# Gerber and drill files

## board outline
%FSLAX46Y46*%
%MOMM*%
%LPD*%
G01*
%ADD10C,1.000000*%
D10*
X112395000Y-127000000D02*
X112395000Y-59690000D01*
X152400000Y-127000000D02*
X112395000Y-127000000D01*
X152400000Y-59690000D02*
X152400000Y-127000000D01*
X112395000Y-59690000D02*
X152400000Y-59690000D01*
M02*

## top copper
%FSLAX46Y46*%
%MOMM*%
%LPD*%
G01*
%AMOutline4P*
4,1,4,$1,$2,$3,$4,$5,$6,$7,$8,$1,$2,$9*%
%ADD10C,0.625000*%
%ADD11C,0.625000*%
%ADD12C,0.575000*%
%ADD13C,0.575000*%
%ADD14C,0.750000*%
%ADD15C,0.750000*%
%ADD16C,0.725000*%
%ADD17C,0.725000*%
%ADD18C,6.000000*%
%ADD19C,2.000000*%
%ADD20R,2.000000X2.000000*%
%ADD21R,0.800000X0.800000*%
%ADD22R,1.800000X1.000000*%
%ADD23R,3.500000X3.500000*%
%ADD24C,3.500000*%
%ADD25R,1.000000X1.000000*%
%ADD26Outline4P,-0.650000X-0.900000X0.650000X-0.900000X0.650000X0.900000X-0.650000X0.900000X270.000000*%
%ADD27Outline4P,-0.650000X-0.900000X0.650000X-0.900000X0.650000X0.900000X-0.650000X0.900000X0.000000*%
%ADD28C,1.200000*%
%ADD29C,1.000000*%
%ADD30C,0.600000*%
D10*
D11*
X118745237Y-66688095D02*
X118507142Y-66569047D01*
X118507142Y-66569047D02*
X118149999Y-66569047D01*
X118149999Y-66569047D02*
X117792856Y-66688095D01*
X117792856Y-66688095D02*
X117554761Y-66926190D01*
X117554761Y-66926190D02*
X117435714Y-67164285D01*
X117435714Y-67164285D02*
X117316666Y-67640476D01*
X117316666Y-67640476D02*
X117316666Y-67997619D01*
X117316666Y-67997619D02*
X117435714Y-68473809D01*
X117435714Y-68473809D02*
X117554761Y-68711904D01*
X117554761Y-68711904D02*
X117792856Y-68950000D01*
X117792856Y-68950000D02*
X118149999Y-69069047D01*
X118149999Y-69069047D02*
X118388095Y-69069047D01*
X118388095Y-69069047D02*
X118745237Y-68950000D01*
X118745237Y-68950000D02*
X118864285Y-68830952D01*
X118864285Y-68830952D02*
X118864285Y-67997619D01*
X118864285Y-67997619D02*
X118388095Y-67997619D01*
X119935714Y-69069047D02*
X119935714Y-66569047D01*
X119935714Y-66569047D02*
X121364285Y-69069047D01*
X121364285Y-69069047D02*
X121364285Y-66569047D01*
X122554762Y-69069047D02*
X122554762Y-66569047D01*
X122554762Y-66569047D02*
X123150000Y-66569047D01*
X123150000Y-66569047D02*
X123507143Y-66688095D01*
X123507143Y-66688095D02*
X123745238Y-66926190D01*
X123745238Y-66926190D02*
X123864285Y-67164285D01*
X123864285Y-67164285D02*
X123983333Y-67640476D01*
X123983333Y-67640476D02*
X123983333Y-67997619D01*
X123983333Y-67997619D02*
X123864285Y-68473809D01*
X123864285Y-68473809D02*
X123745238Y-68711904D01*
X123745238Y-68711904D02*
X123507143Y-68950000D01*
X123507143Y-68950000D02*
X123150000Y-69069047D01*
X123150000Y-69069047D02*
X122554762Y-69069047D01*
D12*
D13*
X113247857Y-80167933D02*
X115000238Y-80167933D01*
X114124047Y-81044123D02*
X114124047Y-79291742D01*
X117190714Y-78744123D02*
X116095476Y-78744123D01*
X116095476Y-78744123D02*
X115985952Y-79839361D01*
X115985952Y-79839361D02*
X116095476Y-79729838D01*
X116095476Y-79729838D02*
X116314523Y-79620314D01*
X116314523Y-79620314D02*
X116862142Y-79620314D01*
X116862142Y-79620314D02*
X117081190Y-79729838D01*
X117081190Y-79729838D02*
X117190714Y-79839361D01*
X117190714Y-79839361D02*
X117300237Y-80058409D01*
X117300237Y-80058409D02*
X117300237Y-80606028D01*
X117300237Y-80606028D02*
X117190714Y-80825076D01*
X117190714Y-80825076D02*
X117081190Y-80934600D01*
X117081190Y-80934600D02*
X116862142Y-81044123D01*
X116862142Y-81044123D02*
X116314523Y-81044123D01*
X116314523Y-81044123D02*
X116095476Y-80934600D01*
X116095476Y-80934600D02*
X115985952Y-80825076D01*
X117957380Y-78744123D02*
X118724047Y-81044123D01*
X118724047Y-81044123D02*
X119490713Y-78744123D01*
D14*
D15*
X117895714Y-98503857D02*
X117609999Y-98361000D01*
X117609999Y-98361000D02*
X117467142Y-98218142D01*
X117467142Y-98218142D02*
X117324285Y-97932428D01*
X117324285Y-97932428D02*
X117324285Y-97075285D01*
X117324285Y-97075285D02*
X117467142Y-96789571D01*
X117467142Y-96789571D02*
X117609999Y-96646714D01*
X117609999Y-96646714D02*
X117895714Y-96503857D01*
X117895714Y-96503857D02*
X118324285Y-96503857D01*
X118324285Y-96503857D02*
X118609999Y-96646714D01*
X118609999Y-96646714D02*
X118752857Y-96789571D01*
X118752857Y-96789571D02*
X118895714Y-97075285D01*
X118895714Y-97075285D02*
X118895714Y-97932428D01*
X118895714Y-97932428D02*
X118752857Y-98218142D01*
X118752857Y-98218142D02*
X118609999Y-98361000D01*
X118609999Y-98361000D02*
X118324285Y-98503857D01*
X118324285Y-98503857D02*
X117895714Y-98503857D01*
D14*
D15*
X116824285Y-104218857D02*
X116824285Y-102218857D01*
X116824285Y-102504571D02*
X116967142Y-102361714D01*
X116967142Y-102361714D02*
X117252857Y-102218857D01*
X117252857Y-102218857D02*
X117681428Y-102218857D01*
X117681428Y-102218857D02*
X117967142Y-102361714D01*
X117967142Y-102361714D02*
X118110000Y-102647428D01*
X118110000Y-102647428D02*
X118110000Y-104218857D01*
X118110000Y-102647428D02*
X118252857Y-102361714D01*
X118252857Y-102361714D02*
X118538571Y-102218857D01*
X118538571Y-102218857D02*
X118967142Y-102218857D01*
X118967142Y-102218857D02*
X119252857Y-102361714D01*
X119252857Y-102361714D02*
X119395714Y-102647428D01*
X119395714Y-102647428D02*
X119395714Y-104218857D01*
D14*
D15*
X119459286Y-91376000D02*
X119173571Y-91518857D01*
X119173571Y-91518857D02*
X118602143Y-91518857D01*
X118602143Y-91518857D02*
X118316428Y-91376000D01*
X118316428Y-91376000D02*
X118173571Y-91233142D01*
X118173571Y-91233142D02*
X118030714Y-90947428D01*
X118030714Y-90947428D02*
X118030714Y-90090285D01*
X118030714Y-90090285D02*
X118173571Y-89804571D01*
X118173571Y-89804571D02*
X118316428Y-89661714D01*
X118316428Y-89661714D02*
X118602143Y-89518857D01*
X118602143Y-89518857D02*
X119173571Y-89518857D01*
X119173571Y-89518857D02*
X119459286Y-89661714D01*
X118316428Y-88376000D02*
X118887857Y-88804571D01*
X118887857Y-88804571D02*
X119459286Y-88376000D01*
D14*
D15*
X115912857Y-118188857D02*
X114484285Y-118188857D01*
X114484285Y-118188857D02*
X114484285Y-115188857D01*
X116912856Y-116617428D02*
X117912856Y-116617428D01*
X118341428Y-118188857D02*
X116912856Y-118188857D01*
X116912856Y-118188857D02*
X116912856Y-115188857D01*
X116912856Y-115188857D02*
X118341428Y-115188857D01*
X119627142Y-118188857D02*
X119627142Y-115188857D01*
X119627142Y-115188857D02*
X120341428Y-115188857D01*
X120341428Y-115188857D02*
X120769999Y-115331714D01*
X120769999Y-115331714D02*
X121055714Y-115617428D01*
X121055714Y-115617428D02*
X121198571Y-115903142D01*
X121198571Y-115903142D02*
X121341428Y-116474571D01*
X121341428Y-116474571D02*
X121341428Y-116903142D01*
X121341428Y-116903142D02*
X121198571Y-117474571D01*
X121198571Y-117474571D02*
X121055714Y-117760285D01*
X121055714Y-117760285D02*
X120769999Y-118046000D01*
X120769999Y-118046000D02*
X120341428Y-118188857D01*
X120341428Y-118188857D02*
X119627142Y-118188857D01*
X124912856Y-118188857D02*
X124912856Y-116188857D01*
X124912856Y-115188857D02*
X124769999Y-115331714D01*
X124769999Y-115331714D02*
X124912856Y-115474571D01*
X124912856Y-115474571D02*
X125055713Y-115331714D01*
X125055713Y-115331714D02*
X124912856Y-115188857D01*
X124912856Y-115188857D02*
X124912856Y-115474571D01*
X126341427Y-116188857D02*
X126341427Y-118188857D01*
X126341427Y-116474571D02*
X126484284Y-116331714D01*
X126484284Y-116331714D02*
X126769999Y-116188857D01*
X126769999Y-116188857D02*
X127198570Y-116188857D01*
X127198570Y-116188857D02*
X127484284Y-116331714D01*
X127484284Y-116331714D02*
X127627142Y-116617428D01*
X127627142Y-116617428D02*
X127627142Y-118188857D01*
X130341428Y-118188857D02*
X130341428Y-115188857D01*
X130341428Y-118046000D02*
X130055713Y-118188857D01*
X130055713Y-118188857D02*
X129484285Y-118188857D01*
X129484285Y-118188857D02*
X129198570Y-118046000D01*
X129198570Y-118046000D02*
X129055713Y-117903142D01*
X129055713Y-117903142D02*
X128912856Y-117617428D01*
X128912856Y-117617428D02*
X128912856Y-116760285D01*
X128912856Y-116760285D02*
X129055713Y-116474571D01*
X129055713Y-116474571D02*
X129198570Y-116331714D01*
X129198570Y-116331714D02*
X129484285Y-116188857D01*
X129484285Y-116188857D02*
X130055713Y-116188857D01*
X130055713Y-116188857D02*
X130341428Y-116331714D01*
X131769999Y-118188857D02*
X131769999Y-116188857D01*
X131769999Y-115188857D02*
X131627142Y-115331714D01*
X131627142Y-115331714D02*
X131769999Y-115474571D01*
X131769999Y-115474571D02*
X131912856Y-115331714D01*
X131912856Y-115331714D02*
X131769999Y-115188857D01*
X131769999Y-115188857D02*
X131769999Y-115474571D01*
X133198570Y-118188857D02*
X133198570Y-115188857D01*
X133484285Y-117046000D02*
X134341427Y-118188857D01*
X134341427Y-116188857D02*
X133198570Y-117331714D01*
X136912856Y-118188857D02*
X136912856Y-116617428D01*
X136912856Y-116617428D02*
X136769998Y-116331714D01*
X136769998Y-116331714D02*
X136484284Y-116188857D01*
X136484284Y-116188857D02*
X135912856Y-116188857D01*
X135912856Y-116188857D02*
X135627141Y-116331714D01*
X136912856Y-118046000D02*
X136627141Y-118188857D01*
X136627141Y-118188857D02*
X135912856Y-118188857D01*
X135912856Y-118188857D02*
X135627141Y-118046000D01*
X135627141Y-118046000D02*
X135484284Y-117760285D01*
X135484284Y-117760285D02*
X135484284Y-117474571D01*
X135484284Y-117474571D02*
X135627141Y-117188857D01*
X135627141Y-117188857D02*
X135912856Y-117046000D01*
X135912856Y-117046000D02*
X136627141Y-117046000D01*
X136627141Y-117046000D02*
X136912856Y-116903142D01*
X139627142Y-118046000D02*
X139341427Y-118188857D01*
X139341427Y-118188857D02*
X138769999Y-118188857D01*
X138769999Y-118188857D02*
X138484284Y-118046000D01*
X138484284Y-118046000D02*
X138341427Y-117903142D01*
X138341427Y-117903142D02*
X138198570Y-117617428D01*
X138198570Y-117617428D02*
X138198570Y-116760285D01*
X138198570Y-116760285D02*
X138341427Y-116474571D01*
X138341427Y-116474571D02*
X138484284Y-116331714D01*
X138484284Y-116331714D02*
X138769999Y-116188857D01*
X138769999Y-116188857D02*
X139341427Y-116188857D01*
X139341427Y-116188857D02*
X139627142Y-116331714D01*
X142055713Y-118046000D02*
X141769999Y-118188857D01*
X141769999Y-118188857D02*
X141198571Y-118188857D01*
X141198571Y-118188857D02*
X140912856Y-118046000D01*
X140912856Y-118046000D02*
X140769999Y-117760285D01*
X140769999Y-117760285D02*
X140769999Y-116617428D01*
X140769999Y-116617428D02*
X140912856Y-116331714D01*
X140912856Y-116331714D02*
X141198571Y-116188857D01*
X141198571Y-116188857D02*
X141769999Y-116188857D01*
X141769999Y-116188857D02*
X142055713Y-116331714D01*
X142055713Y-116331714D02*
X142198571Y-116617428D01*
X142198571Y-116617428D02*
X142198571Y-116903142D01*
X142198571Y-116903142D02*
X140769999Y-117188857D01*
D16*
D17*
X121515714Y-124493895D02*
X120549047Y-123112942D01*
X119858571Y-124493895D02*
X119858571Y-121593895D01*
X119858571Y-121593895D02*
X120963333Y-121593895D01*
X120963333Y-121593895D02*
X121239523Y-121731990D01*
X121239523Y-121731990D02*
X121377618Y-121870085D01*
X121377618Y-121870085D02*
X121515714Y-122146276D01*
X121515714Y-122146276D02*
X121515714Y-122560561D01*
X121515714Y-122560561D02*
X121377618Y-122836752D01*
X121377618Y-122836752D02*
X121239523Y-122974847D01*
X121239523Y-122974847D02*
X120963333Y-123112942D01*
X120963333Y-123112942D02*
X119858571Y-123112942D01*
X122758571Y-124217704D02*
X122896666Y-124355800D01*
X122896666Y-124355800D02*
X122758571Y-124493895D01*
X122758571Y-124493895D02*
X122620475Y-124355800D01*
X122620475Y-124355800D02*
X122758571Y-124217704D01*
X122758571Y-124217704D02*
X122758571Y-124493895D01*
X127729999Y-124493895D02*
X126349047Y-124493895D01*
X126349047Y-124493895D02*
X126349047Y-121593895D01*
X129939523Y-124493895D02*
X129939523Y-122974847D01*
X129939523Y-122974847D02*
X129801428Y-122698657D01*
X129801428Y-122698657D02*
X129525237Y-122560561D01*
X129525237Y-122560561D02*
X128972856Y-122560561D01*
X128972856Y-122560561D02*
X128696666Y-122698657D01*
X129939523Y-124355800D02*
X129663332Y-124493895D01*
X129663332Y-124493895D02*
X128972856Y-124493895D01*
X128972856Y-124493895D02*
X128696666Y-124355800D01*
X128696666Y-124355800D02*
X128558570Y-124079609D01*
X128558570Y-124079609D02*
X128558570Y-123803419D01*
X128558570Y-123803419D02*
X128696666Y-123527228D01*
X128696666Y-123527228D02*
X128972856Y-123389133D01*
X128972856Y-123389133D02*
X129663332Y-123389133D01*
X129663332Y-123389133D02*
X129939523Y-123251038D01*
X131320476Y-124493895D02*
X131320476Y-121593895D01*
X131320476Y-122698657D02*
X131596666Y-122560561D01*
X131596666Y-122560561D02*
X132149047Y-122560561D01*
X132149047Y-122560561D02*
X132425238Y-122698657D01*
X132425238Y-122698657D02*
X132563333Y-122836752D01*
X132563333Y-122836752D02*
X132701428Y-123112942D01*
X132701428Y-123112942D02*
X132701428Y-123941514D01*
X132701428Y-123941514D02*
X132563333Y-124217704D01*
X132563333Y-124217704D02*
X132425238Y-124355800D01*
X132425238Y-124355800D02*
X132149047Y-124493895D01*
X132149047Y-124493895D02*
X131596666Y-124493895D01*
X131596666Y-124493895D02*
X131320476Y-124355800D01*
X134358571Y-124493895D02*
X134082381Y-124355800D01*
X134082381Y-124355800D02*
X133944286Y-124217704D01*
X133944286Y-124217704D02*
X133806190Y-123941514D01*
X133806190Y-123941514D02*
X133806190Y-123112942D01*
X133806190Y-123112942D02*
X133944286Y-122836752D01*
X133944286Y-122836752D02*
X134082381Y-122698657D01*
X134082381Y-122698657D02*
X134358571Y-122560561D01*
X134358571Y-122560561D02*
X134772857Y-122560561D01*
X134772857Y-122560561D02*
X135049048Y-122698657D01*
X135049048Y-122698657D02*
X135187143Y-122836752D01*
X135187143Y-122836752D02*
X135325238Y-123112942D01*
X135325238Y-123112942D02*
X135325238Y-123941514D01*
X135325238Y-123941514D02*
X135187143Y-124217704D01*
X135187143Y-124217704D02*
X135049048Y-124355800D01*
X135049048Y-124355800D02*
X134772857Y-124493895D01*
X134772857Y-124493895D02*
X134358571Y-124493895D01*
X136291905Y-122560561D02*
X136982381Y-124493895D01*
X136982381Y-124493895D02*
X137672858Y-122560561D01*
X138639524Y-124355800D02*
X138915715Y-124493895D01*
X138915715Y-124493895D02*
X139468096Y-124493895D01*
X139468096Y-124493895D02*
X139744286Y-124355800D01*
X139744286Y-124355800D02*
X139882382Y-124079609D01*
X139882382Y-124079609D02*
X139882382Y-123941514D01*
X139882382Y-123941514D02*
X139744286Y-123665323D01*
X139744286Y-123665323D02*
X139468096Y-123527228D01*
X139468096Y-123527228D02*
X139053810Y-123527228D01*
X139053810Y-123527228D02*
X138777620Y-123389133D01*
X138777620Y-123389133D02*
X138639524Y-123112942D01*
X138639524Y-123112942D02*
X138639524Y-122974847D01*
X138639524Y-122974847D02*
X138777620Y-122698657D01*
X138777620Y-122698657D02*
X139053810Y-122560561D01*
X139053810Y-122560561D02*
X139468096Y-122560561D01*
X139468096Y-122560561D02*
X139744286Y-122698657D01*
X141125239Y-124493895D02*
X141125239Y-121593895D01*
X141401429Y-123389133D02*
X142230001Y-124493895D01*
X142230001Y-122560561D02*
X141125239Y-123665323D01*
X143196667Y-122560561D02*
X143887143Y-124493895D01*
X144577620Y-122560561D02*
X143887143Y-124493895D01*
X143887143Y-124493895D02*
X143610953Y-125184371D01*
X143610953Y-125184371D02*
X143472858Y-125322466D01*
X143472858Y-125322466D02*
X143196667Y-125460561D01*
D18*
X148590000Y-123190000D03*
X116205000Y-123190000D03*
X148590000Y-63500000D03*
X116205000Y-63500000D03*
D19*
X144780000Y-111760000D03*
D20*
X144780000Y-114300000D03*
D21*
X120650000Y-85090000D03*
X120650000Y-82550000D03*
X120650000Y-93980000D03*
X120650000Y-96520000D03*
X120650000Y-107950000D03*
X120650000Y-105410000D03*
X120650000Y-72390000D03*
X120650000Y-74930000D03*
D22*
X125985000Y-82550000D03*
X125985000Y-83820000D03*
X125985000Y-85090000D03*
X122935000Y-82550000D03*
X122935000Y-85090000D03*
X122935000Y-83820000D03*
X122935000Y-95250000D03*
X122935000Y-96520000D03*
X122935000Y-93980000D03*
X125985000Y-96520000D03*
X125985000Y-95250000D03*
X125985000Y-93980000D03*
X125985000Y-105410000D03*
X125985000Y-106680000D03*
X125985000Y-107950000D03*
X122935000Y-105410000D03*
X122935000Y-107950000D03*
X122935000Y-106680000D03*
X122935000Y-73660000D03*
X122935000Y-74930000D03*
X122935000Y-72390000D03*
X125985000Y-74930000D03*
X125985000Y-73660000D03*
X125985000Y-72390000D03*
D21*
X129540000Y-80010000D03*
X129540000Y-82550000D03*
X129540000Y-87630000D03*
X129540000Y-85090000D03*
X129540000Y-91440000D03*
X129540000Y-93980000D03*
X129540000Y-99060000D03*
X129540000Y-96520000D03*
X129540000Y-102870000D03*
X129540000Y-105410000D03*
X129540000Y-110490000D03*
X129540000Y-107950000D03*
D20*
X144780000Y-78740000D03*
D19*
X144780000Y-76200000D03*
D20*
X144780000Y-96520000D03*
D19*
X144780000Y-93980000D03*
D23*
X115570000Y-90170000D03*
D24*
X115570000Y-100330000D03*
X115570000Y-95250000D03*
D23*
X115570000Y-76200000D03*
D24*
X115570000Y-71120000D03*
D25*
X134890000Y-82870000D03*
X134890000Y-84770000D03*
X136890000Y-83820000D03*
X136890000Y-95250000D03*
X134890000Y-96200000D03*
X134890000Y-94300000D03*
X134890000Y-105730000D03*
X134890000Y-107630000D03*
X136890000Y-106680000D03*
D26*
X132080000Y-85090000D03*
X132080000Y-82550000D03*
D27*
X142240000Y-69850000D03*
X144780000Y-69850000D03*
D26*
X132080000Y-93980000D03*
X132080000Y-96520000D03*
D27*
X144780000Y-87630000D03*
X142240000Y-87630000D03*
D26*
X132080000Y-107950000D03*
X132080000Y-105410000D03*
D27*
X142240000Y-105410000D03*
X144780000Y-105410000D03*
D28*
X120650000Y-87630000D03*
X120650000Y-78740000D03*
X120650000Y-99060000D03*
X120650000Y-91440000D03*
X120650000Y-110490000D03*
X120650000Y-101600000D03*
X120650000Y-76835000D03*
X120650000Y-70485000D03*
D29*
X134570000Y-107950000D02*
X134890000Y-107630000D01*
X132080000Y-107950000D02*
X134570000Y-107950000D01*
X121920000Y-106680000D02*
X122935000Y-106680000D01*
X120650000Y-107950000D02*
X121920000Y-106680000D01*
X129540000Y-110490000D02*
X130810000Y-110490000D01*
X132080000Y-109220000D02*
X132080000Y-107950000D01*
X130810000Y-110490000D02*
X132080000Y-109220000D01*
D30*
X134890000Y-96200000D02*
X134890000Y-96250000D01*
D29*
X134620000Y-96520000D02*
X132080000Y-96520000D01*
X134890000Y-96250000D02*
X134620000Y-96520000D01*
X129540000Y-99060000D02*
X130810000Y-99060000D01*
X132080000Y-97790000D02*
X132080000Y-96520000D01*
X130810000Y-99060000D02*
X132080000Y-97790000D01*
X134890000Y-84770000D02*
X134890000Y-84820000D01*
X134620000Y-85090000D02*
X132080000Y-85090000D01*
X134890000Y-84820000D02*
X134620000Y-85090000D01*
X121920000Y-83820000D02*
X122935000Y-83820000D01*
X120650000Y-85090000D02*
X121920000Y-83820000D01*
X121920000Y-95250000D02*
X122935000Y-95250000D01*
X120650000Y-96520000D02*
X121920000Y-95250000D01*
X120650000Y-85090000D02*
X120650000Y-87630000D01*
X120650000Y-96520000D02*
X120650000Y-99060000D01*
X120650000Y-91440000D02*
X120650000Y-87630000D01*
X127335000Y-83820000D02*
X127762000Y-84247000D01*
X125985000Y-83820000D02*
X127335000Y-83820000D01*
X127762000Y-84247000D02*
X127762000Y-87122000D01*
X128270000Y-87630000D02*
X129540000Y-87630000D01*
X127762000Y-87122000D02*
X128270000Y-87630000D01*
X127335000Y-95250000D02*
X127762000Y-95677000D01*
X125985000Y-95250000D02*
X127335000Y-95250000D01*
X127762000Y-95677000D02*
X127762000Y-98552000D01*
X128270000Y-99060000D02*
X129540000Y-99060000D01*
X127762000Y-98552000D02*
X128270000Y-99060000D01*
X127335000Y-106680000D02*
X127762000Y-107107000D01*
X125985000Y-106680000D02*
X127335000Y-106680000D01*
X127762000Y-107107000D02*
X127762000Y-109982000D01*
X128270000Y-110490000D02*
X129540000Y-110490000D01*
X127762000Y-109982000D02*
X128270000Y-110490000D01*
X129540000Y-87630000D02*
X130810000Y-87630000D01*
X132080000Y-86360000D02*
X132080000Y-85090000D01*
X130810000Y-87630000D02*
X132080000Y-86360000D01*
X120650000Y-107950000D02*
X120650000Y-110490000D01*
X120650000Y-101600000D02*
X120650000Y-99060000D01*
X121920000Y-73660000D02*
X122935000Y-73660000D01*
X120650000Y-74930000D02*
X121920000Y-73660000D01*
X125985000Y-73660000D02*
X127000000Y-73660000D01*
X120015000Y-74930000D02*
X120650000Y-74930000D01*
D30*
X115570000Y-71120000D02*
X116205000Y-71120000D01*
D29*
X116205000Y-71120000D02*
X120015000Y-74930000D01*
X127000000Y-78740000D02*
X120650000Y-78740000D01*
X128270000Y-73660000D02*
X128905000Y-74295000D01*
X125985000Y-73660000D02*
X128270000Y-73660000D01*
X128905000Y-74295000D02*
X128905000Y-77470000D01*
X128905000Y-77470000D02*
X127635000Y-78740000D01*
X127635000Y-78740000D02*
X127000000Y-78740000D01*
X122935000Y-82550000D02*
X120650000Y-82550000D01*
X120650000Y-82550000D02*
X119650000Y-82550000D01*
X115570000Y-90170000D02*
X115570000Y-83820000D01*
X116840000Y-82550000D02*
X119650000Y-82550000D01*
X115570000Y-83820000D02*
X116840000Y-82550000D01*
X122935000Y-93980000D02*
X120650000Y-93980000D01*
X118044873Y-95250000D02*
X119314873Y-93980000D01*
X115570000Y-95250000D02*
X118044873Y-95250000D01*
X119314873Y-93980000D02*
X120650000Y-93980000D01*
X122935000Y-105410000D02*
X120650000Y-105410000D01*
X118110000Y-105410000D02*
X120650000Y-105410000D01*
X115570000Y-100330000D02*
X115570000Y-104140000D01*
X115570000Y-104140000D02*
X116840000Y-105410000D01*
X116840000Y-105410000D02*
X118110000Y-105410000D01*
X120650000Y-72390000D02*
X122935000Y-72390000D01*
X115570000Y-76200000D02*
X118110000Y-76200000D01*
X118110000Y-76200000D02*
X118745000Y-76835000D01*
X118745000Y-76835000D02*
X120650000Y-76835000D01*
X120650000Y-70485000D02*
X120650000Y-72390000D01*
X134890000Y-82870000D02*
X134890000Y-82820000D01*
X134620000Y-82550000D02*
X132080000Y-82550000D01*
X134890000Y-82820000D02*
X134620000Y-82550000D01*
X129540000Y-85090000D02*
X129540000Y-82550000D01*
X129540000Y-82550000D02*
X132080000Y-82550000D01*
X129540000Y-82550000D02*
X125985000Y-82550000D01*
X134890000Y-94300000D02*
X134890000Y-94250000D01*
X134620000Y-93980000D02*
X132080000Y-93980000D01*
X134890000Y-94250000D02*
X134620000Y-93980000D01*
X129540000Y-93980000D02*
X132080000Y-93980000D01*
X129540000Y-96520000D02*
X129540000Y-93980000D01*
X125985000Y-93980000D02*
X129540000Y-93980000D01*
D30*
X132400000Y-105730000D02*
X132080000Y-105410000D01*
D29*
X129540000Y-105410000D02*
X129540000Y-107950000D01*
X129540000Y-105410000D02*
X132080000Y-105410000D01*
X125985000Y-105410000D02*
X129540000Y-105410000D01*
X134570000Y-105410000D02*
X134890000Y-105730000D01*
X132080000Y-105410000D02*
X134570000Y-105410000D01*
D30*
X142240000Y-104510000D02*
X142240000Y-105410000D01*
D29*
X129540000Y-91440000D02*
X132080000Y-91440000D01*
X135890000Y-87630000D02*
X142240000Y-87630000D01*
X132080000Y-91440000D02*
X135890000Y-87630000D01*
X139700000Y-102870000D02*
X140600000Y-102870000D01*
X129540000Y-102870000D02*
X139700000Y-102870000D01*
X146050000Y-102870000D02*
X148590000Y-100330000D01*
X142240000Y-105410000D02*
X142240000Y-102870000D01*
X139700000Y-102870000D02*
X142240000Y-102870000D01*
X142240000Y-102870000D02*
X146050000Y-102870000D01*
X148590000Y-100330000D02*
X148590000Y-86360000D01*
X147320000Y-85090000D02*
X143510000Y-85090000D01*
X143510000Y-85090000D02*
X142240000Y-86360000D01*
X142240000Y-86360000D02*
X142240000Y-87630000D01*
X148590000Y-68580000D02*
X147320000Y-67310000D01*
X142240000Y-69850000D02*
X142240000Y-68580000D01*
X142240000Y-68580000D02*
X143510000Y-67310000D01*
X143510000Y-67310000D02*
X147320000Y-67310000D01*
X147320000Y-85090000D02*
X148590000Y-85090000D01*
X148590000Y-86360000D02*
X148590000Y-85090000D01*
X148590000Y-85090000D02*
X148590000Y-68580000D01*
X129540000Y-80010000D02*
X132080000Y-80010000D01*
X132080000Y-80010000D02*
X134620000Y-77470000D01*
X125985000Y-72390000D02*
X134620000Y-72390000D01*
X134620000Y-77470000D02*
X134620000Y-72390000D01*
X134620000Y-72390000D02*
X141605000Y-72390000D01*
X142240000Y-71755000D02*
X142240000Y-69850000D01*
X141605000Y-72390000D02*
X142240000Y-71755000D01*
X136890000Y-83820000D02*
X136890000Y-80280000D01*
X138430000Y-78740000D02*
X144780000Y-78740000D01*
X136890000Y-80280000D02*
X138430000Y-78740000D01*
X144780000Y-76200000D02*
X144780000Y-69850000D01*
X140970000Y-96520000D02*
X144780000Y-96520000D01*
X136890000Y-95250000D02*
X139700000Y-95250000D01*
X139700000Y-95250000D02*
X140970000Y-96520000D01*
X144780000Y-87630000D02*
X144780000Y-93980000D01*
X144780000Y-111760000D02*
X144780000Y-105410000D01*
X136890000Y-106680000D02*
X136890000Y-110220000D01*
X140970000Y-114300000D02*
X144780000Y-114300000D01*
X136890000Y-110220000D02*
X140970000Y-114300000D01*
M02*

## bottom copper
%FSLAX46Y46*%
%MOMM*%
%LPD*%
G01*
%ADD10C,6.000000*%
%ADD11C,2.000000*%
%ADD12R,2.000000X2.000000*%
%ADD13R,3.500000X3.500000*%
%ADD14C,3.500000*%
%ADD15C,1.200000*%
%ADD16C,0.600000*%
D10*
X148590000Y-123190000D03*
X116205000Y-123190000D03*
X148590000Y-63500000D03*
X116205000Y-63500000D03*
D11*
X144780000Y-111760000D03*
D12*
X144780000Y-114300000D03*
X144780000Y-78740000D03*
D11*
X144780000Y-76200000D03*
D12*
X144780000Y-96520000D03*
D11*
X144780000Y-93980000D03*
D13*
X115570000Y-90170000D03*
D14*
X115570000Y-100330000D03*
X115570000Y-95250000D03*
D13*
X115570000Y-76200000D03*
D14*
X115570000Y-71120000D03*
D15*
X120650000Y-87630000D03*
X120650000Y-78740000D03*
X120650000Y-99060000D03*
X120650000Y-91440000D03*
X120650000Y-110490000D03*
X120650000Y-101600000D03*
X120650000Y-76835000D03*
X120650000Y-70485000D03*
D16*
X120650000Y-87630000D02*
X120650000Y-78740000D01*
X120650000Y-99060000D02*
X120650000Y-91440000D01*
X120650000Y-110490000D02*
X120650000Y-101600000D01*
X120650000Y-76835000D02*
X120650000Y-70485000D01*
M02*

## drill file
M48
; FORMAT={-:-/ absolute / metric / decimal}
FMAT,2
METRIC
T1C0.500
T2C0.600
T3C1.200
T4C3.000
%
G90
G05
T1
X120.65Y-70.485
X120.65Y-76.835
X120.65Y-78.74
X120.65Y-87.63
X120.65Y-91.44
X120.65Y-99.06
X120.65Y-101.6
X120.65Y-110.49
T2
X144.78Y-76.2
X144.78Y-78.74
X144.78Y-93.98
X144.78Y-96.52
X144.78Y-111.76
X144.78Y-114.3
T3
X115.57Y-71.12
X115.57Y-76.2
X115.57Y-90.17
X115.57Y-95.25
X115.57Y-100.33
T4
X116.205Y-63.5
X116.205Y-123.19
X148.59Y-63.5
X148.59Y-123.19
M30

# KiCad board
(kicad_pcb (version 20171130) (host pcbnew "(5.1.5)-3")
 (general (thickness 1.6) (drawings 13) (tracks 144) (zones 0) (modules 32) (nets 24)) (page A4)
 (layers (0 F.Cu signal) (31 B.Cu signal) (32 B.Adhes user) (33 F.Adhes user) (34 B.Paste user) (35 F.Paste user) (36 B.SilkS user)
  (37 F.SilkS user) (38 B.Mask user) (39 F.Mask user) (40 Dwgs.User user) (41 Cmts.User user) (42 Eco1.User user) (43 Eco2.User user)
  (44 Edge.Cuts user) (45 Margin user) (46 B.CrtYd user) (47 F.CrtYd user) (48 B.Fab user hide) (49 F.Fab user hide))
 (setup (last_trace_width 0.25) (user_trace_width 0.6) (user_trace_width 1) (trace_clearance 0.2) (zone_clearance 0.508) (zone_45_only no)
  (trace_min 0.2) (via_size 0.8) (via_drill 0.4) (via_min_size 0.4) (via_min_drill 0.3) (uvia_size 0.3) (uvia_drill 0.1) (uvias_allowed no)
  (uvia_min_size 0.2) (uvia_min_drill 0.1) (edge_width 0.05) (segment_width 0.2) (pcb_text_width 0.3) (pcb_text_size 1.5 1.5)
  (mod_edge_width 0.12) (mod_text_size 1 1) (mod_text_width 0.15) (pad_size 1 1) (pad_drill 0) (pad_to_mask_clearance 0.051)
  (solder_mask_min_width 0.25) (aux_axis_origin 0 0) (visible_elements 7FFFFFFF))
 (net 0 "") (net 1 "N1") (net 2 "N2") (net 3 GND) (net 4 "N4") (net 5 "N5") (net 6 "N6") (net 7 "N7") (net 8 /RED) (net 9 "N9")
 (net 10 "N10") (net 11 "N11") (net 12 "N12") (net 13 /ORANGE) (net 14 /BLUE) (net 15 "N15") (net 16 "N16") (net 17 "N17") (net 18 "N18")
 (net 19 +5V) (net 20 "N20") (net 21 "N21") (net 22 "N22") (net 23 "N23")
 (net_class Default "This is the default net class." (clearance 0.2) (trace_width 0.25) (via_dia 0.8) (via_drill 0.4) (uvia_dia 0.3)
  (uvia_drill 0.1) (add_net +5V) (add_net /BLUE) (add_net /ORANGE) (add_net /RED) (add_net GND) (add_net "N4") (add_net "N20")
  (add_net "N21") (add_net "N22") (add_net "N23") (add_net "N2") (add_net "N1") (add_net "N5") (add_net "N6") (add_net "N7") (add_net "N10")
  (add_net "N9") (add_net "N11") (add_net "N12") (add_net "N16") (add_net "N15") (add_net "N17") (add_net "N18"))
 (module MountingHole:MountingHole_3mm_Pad (layer F.Cu) (at 148.59 123.19)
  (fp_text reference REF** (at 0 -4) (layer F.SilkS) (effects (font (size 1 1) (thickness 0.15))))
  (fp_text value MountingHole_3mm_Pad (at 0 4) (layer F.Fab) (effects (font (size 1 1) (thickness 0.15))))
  (pad 4 thru_hole circle (at 0 0) (size 6 6) (drill 3) (layers *.Cu *.Mask)))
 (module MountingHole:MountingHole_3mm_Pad (layer F.Cu) (at 116.205 123.19)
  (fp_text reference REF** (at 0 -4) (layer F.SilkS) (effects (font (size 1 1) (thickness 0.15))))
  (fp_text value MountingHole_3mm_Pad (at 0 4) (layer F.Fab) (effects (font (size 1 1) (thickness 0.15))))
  (pad 3 thru_hole circle (at 0 0) (size 6 6) (drill 3) (layers *.Cu *.Mask)))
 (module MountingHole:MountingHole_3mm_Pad (layer F.Cu) (at 148.59 63.5)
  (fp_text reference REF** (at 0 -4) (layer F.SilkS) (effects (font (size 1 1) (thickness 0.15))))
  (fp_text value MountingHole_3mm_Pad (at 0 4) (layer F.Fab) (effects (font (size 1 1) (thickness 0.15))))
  (pad 2 thru_hole circle (at 0 0) (size 6 6) (drill 3) (layers *.Cu *.Mask)))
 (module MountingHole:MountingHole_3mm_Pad (layer F.Cu) (at 116.205 63.5)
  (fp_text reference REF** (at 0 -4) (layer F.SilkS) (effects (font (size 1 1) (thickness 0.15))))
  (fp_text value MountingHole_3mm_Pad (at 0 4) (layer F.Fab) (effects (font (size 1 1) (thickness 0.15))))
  (pad 1 thru_hole circle (at 0 0) (size 6 6) (drill 3) (layers *.Cu *.Mask)))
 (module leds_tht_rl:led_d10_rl (layer F.Cu) (at 144.78 113.03 90)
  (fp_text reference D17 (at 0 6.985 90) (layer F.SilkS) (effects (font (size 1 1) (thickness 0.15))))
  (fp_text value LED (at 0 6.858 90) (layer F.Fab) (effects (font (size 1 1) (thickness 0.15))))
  (pad 2 thru_hole circle (at 1.27 0 90) (size 2 2) (drill 0.6) (layers *.Cu *.Mask) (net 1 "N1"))
  (pad 1 thru_hole rect (at -1.27 0 90) (size 2 2) (drill 0.6) (layers *.Cu *.Mask) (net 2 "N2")))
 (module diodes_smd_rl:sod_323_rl (layer F.Cu) (at 120.65 83.82 270)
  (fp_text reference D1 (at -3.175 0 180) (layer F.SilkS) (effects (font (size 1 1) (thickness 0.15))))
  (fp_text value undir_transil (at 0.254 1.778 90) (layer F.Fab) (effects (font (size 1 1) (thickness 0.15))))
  (pad 2 smd rect (at 1.27 0 270) (size 0.8 0.8) (layers F.Cu F.Paste F.Mask) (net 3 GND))
  (pad 1 smd rect (at -1.27 0 270) (size 0.8 0.8) (layers F.Cu F.Paste F.Mask) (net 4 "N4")))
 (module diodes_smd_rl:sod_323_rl (layer F.Cu) (at 120.65 95.25 270)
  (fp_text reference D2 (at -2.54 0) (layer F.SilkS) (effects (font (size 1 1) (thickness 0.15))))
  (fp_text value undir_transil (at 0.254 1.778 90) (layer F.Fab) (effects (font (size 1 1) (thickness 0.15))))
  (pad 1 smd rect (at -1.27 0 270) (size 0.8 0.8) (layers F.Cu F.Paste F.Mask) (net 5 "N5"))
  (pad 2 smd rect (at 1.27 0 270) (size 0.8 0.8) (layers F.Cu F.Paste F.Mask) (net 3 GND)))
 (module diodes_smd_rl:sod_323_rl (layer F.Cu) (at 120.65 106.68 270)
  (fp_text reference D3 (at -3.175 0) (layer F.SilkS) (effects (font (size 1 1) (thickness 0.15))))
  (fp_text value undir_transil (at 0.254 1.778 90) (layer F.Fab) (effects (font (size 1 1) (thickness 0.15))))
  (pad 2 smd rect (at 1.27 0 270) (size 0.8 0.8) (layers F.Cu F.Paste F.Mask) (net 3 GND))
  (pad 1 smd rect (at -1.27 0 270) (size 0.8 0.8) (layers F.Cu F.Paste F.Mask) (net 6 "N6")))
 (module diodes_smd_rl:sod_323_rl (layer F.Cu) (at 120.65 73.66 270)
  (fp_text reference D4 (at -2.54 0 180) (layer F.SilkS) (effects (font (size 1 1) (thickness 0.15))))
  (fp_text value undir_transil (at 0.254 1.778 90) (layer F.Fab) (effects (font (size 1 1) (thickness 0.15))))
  (pad 1 smd rect (at -1.27 0 270) (size 0.8 0.8) (layers F.Cu F.Paste F.Mask) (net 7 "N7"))
  (pad 2 smd rect (at 1.27 0 270) (size 0.8 0.8) (layers F.Cu F.Paste F.Mask) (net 3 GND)))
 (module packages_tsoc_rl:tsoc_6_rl (layer F.Cu) (at 124.46 83.82)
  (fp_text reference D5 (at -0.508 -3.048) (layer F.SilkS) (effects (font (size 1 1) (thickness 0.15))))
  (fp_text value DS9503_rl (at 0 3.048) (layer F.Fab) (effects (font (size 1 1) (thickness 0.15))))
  (pad 6 smd rect (at 1.525 -1.27) (size 1.8 1) (layers F.Cu F.Paste F.Mask) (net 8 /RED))
  (pad 5 smd rect (at 1.525 0) (size 1.8 1) (layers F.Cu F.Paste F.Mask) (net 3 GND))
  (pad 4 smd rect (at 1.525 1.27) (size 1.8 1) (layers F.Cu F.Paste F.Mask) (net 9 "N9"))
  (pad 1 smd rect (at -1.525 -1.27) (size 1.8 1) (layers F.Cu F.Paste F.Mask) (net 4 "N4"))
  (pad 3 smd rect (at -1.525 1.27) (size 1.8 1) (layers F.Cu F.Paste F.Mask) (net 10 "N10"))
  (pad 2 smd rect (at -1.525 0) (size 1.8 1) (layers F.Cu F.Paste F.Mask) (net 3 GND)))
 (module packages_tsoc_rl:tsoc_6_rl (layer F.Cu) (at 124.46 95.25)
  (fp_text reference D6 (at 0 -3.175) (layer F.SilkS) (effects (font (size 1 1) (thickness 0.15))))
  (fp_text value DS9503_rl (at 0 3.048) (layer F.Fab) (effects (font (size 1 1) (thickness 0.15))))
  (pad 2 smd rect (at -1.525 0) (size 1.8 1) (layers F.Cu F.Paste F.Mask) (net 3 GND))
  (pad 3 smd rect (at -1.525 1.27) (size 1.8 1) (layers F.Cu F.Paste F.Mask) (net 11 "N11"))
  (pad 1 smd rect (at -1.525 -1.27) (size 1.8 1) (layers F.Cu F.Paste F.Mask) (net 5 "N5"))
  (pad 4 smd rect (at 1.525 1.27) (size 1.8 1) (layers F.Cu F.Paste F.Mask) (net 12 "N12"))
  (pad 5 smd rect (at 1.525 0) (size 1.8 1) (layers F.Cu F.Paste F.Mask) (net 3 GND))
  (pad 6 smd rect (at 1.525 -1.27) (size 1.8 1) (layers F.Cu F.Paste F.Mask) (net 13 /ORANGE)))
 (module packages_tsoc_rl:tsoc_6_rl (layer F.Cu) (at 124.46 106.68)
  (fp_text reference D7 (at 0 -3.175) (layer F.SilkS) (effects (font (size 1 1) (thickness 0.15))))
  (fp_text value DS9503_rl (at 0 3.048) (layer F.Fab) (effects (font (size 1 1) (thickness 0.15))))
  (pad 6 smd rect (at 1.525 -1.27) (size 1.8 1) (layers F.Cu F.Paste F.Mask) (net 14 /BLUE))
  (pad 5 smd rect (at 1.525 0) (size 1.8 1) (layers F.Cu F.Paste F.Mask) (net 3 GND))
  (pad 4 smd rect (at 1.525 1.27) (size 1.8 1) (layers F.Cu F.Paste F.Mask) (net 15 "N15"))
  (pad 1 smd rect (at -1.525 -1.27) (size 1.8 1) (layers F.Cu F.Paste F.Mask) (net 6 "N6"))
  (pad 3 smd rect (at -1.525 1.27) (size 1.8 1) (layers F.Cu F.Paste F.Mask) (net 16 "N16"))
  (pad 2 smd rect (at -1.525 0) (size 1.8 1) (layers F.Cu F.Paste F.Mask) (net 3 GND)))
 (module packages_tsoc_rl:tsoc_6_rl (layer F.Cu) (at 124.46 73.66)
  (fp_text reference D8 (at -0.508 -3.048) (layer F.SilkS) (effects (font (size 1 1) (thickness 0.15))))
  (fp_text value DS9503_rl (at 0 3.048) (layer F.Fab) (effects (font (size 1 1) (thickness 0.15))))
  (pad 2 smd rect (at -1.525 0) (size 1.8 1) (layers F.Cu F.Paste F.Mask) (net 3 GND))
  (pad 3 smd rect (at -1.525 1.27) (size 1.8 1) (layers F.Cu F.Paste F.Mask) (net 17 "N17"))
  (pad 1 smd rect (at -1.525 -1.27) (size 1.8 1) (layers F.Cu F.Paste F.Mask) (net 7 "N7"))
  (pad 4 smd rect (at 1.525 1.27) (size 1.8 1) (layers F.Cu F.Paste F.Mask) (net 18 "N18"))
  (pad 5 smd rect (at 1.525 0) (size 1.8 1) (layers F.Cu F.Paste F.Mask) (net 3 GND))
  (pad 6 smd rect (at 1.525 -1.27) (size 1.8 1) (layers F.Cu F.Paste F.Mask) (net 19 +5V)))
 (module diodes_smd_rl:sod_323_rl (layer F.Cu) (at 129.54 81.28 270)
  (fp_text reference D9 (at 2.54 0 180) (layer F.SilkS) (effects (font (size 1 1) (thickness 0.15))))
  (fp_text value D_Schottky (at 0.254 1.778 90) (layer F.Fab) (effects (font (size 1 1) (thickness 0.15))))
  (pad 1 smd rect (at -1.27 0 270) (size 0.8 0.8) (layers F.Cu F.Paste F.Mask) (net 19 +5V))
  (pad 2 smd rect (at 1.27 0 270) (size 0.8 0.8) (layers F.Cu F.Paste F.Mask) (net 8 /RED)))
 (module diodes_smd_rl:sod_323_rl (layer F.Cu) (at 129.54 86.36 270)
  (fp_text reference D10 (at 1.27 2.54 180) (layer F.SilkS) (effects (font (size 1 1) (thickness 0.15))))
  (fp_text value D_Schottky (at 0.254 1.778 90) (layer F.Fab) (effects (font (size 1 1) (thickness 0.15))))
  (pad 2 smd rect (at 1.27 0 270) (size 0.8 0.8) (layers F.Cu F.Paste F.Mask) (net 3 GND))
  (pad 1 smd rect (at -1.27 0 270) (size 0.8 0.8) (layers F.Cu F.Paste F.Mask) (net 8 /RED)))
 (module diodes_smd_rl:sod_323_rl (layer F.Cu) (at 129.54 92.71 270)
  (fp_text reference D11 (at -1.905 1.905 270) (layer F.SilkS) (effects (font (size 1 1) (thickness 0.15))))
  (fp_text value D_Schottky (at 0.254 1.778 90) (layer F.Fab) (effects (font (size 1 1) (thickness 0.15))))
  (pad 1 smd rect (at -1.27 0 270) (size 0.8 0.8) (layers F.Cu F.Paste F.Mask) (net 19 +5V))
  (pad 2 smd rect (at 1.27 0 270) (size 0.8 0.8) (layers F.Cu F.Paste F.Mask) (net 13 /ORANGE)))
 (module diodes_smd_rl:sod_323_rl (layer F.Cu) (at 129.54 97.79 270)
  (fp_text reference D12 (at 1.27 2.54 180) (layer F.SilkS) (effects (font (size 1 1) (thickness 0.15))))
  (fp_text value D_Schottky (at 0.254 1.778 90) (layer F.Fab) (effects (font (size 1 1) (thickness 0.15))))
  (pad 2 smd rect (at 1.27 0 270) (size 0.8 0.8) (layers F.Cu F.Paste F.Mask) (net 3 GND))
  (pad 1 smd rect (at -1.27 0 270) (size 0.8 0.8) (layers F.Cu F.Paste F.Mask) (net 13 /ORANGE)))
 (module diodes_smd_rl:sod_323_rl (layer F.Cu) (at 129.54 104.14 270)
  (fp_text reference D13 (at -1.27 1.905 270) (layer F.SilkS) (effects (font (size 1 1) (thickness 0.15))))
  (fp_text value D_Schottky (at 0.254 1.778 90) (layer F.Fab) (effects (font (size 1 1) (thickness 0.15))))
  (pad 1 smd rect (at -1.27 0 270) (size 0.8 0.8) (layers F.Cu F.Paste F.Mask) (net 19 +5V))
  (pad 2 smd rect (at 1.27 0 270) (size 0.8 0.8) (layers F.Cu F.Paste F.Mask) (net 14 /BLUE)))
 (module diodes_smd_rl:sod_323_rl (layer F.Cu) (at 129.54 109.22 270)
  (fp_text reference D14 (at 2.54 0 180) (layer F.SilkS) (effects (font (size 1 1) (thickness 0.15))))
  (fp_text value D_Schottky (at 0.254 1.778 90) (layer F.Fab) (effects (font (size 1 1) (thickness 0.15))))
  (pad 2 smd rect (at 1.27 0 270) (size 0.8 0.8) (layers F.Cu F.Paste F.Mask) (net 3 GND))
  (pad 1 smd rect (at -1.27 0 270) (size 0.8 0.8) (layers F.Cu F.Paste F.Mask) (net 14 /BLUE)))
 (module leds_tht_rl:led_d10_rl (layer F.Cu) (at 144.78 77.47 90)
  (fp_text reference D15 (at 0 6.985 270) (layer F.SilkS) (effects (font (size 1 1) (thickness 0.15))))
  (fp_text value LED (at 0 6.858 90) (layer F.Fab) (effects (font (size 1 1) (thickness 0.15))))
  (pad 1 thru_hole rect (at -1.27 0 90) (size 2 2) (drill 0.6) (layers *.Cu *.Mask) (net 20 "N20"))
  (pad 2 thru_hole circle (at 1.27 0 90) (size 2 2) (drill 0.6) (layers *.Cu *.Mask) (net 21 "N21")))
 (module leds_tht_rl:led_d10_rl (layer F.Cu) (at 144.78 95.25 90)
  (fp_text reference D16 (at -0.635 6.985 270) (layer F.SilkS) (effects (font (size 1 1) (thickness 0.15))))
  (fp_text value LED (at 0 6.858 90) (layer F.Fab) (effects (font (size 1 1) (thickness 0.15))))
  (pad 1 thru_hole rect (at -1.27 0 90) (size 2 2) (drill 0.6) (layers *.Cu *.Mask) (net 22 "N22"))
  (pad 2 thru_hole circle (at 1.27 0 90) (size 2 2) (drill 0.6) (layers *.Cu *.Mask) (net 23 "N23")))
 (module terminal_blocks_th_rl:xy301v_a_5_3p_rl (layer F.Cu) (at 115.57 95.25 270)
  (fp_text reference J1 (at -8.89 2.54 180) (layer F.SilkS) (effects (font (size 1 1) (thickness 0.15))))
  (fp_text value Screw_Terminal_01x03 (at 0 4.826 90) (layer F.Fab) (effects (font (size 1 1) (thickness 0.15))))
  (pad 1 thru_hole rect (at -5.08 0 270) (size 3.5 3.5) (drill 1.2) (layers *.Cu *.Mask) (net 4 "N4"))
  (pad 3 thru_hole circle (at 5.08 0 270) (size 3.5 3.5) (drill 1.2) (layers *.Cu *.Mask) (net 6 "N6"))
  (pad 2 thru_hole circle (at 0 0 270) (size 3.5 3.5) (drill 1.2) (layers *.Cu *.Mask) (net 5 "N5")))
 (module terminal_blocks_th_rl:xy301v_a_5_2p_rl (layer B.Cu) (at 115.57 73.66 90)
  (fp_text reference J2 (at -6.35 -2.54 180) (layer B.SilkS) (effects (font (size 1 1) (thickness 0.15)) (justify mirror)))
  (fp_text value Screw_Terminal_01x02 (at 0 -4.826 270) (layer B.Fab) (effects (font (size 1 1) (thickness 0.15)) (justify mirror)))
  (pad 1 thru_hole rect (at -2.54 0 90) (size 3.5 3.5) (drill 1.2) (layers *.Cu *.Mask) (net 7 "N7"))
  (pad 2 thru_hole circle (at 2.54 0 90) (size 3.5 3.5) (drill 1.2) (layers *.Cu *.Mask) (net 3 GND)))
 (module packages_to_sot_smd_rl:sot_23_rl (layer F.Cu) (at 135.89 83.82)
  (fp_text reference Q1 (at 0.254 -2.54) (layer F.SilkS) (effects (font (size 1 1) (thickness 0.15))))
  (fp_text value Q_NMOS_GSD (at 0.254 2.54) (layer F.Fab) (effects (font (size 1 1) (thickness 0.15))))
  (pad 1 smd rect (at -1 -0.95) (size 1 1) (layers F.Cu F.Paste F.Mask) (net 8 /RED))
  (pad 2 smd rect (at -1 0.95) (size 1 1) (layers F.Cu F.Paste F.Mask) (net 3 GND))
  (pad 3 smd rect (at 1 0) (size 1 1) (layers F.Cu F.Paste F.Mask) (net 20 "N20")))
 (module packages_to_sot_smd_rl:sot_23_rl (layer F.Cu) (at 135.89 95.25)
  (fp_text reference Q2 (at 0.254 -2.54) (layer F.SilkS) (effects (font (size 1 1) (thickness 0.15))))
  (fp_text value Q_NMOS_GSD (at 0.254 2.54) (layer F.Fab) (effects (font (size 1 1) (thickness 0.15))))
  (pad 3 smd rect (at 1 0) (size 1 1) (layers F.Cu F.Paste F.Mask) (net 22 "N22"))
  (pad 2 smd rect (at -1 0.95) (size 1 1) (layers F.Cu F.Paste F.Mask) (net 3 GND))
  (pad 1 smd rect (at -1 -0.95) (size 1 1) (layers F.Cu F.Paste F.Mask) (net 13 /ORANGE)))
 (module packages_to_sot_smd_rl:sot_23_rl (layer F.Cu) (at 135.89 106.68)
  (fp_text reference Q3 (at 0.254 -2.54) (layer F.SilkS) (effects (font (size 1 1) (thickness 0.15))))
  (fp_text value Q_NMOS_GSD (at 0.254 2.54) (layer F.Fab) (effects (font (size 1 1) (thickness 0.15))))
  (pad 1 smd rect (at -1 -0.95) (size 1 1) (layers F.Cu F.Paste F.Mask) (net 14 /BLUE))
  (pad 2 smd rect (at -1 0.95) (size 1 1) (layers F.Cu F.Paste F.Mask) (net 3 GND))
  (pad 3 smd rect (at 1 0) (size 1 1) (layers F.Cu F.Paste F.Mask) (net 2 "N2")))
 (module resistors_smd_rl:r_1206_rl (layer F.Cu) (at 132.08 83.82 270)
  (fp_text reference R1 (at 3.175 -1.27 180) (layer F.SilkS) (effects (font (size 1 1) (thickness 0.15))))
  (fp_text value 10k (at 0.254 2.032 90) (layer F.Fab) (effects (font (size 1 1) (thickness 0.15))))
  (pad 2 smd trapezoid (at 1.27 0 270) (size 1.3 1.8) (layers F.Cu F.Paste F.Mask) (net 3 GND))
  (pad 1 smd trapezoid (at -1.27 0 270) (size 1.3 1.8) (layers F.Cu F.Paste F.Mask) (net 8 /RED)))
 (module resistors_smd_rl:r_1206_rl (layer F.Cu) (at 143.51 69.85)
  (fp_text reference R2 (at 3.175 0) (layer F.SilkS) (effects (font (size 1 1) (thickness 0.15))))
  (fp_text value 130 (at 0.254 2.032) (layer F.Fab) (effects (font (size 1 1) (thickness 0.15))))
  (pad 1 smd trapezoid (at -1.27 0) (size 1.3 1.8) (layers F.Cu F.Paste F.Mask) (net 19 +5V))
  (pad 2 smd trapezoid (at 1.27 0) (size 1.3 1.8) (layers F.Cu F.Paste F.Mask) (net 21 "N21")))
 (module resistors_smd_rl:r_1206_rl (layer F.Cu) (at 132.08 95.25 270)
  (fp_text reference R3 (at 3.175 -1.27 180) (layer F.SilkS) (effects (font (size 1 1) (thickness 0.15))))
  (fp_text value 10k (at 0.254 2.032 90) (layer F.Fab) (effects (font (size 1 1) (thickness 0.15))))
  (pad 1 smd trapezoid (at -1.27 0 270) (size 1.3 1.8) (layers F.Cu F.Paste F.Mask) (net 13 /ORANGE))
  (pad 2 smd trapezoid (at 1.27 0 270) (size 1.3 1.8) (layers F.Cu F.Paste F.Mask) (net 3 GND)))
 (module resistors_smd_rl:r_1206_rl (layer F.Cu) (at 143.51 87.63)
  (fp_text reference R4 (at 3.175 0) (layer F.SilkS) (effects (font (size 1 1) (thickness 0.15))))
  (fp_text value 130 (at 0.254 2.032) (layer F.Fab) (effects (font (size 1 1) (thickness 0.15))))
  (pad 2 smd trapezoid (at 1.27 0) (size 1.3 1.8) (layers F.Cu F.Paste F.Mask) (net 23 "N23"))
  (pad 1 smd trapezoid (at -1.27 0) (size 1.3 1.8) (layers F.Cu F.Paste F.Mask) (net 19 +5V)))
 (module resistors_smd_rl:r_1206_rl (layer F.Cu) (at 132.08 106.68 270)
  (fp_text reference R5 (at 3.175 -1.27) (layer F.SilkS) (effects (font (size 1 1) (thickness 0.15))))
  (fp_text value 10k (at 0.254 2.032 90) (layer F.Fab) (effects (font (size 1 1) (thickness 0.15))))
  (pad 2 smd trapezoid (at 1.27 0 270) (size 1.3 1.8) (layers F.Cu F.Paste F.Mask) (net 3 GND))
  (pad 1 smd trapezoid (at -1.27 0 270) (size 1.3 1.8) (layers F.Cu F.Paste F.Mask) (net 14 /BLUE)))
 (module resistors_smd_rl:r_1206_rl (layer F.Cu) (at 143.51 105.41)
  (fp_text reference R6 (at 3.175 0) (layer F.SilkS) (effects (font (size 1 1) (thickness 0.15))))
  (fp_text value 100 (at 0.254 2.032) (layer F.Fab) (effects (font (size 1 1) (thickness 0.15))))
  (pad 1 smd trapezoid (at -1.27 0) (size 1.3 1.8) (layers F.Cu F.Paste F.Mask) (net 19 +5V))
  (pad 2 smd trapezoid (at 1.27 0) (size 1.3 1.8) (layers F.Cu F.Paste F.Mask) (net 1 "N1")))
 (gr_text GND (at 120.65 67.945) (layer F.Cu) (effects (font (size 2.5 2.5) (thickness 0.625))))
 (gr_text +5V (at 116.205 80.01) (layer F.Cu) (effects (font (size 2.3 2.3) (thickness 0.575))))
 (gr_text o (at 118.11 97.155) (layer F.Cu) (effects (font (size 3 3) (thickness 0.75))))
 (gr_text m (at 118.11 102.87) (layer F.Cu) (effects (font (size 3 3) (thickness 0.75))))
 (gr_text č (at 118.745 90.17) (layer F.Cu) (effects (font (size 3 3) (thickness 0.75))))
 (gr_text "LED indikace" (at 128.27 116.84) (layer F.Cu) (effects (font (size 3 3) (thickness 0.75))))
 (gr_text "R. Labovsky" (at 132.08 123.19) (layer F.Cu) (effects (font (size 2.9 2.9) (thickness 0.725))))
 (gr_line (start 112.395 127) (end 112.395 59.69) (layer Edge.Cuts) (width 1))
 (gr_line (start 152.4 127) (end 112.395 127) (layer Edge.Cuts) (width 1))
 (gr_line (start 152.4 59.69) (end 152.4 127) (layer Edge.Cuts) (width 1))
 (gr_line (start 112.395 59.69) (end 152.4 59.69) (layer Edge.Cuts) (width 1))
 (segment (start 134.57 107.95) (end 134.89 107.63) (width 1) (layer F.Cu) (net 3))
 (segment (start 132.08 107.95) (end 134.57 107.95) (width 1) (layer F.Cu) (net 3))
 (segment (start 121.92 106.68) (end 122.935 106.68) (width 1) (layer F.Cu) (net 3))
 (segment (start 120.65 107.95) (end 121.92 106.68) (width 1) (layer F.Cu) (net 3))
 (segment (start 129.54 110.49) (end 130.81 110.49) (width 1) (layer F.Cu) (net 3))
 (segment (start 132.08 109.22) (end 132.08 107.95) (width 1) (layer F.Cu) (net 3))
 (segment (start 130.81 110.49) (end 132.08 109.22) (width 1) (layer F.Cu) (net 3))
 (segment (start 134.89 96.2) (end 134.89 96.25) (width 0.6) (layer F.Cu) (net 3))
 (segment (start 134.62 96.52) (end 132.08 96.52) (width 1) (layer F.Cu) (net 3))
 (segment (start 134.89 96.25) (end 134.62 96.52) (width 1) (layer F.Cu) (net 3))
 (segment (start 129.54 99.06) (end 130.81 99.06) (width 1) (layer F.Cu) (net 3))
 (segment (start 132.08 97.79) (end 132.08 96.52) (width 1) (layer F.Cu) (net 3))
 (segment (start 130.81 99.06) (end 132.08 97.79) (width 1) (layer F.Cu) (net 3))
 (segment (start 134.89 84.77) (end 134.89 84.82) (width 1) (layer F.Cu) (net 3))
 (segment (start 134.62 85.09) (end 132.08 85.09) (width 1) (layer F.Cu) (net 3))
 (segment (start 134.89 84.82) (end 134.62 85.09) (width 1) (layer F.Cu) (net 3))
 (segment (start 121.92 83.82) (end 122.935 83.82) (width 1) (layer F.Cu) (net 3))
 (segment (start 120.65 85.09) (end 121.92 83.82) (width 1) (layer F.Cu) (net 3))
 (segment (start 121.92 95.25) (end 122.935 95.25) (width 1) (layer F.Cu) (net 3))
 (segment (start 120.65 96.52) (end 121.92 95.25) (width 1) (layer F.Cu) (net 3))
 (segment (start 120.65 85.09) (end 120.65 87.63) (width 1) (layer F.Cu) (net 3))
 (via (at 120.65 87.63) (size 1.2) (drill 0.5) (layers F.Cu B.Cu) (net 3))
 (via (at 120.65 78.74) (size 1.2) (drill 0.5) (layers F.Cu B.Cu) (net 3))
 (segment (start 120.65 87.63) (end 120.65 78.74) (width 0.6) (layer B.Cu) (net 3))
 (segment (start 120.65 96.52) (end 120.65 99.06) (width 1) (layer F.Cu) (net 3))
 (via (at 120.65 99.06) (size 1.2) (drill 0.5) (layers F.Cu B.Cu) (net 3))
 (segment (start 120.65 99.06) (end 120.65 91.44) (width 0.6) (layer B.Cu) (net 3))
 (via (at 120.65 91.44) (size 1.2) (drill 0.5) (layers F.Cu B.Cu) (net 3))
 (segment (start 120.65 91.44) (end 120.65 87.63) (width 1) (layer F.Cu) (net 3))
 (segment (start 127.335 83.82) (end 127.762 84.247) (width 1) (layer F.Cu) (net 3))
 (segment (start 125.985 83.82) (end 127.335 83.82) (width 1) (layer F.Cu) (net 3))
 (segment (start 127.762 84.247) (end 127.762 87.122) (width 1) (layer F.Cu) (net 3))
 (segment (start 128.27 87.63) (end 129.54 87.63) (width 1) (layer F.Cu) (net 3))
 (segment (start 127.762 87.122) (end 128.27 87.63) (width 1) (layer F.Cu) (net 3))
 (segment (start 127.335 95.25) (end 127.762 95.677) (width 1) (layer F.Cu) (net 3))
 (segment (start 125.985 95.25) (end 127.335 95.25) (width 1) (layer F.Cu) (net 3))
 (segment (start 127.762 95.677) (end 127.762 98.552) (width 1) (layer F.Cu) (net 3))
 (segment (start 128.27 99.06) (end 129.54 99.06) (width 1) (layer F.Cu) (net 3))
 (segment (start 127.762 98.552) (end 128.27 99.06) (width 1) (layer F.Cu) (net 3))
 (segment (start 127.335 106.68) (end 127.762 107.107) (width 1) (layer F.Cu) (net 3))
 (segment (start 125.985 106.68) (end 127.335 106.68) (width 1) (layer F.Cu) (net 3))
 (segment (start 127.762 107.107) (end 127.762 109.982) (width 1) (layer F.Cu) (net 3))
 (segment (start 128.27 110.49) (end 129.54 110.49) (width 1) (layer F.Cu) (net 3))
 (segment (start 127.762 109.982) (end 128.27 110.49) (width 1) (layer F.Cu) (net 3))
 (segment (start 129.54 87.63) (end 130.81 87.63) (width 1) (layer F.Cu) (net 3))
 (segment (start 132.08 86.36) (end 132.08 85.09) (width 1) (layer F.Cu) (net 3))
 (segment (start 130.81 87.63) (end 132.08 86.36) (width 1) (layer F.Cu) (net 3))
 (segment (start 120.65 107.95) (end 120.65 110.49) (width 1) (layer F.Cu) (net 3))
 (via (at 120.65 110.49) (size 1.2) (drill 0.5) (layers F.Cu B.Cu) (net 3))
 (segment (start 120.65 110.49) (end 120.65 101.6) (width 0.6) (layer B.Cu) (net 3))
 (via (at 120.65 101.6) (size 1.2) (drill 0.5) (layers F.Cu B.Cu) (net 3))
 (segment (start 120.65 101.6) (end 120.65 99.06) (width 1) (layer F.Cu) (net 3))
 (segment (start 121.92 73.66) (end 122.935 73.66) (width 1) (layer F.Cu) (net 3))
 (segment (start 120.65 74.93) (end 121.92 73.66) (width 1) (layer F.Cu) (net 3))
 (segment (start 125.985 73.66) (end 127 73.66) (width 1) (layer F.Cu) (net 3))
 (segment (start 120.015 74.93) (end 120.65 74.93) (width 1) (layer F.Cu) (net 3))
 (segment (start 115.57 71.12) (end 116.205 71.12) (width 0.6) (layer F.Cu) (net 3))
 (segment (start 116.205 71.12) (end 120.015 74.93) (width 1) (layer F.Cu) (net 3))
 (segment (start 127 78.74) (end 120.65 78.74) (width 1) (layer F.Cu) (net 3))
 (segment (start 128.27 73.66) (end 128.905 74.295) (width 1) (layer F.Cu) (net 3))
 (segment (start 125.985 73.66) (end 128.27 73.66) (width 1) (layer F.Cu) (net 3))
 (segment (start 128.905 74.295) (end 128.905 77.47) (width 1) (layer F.Cu) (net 3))
 (segment (start 128.905 77.47) (end 127.635 78.74) (width 1) (layer F.Cu) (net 3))
 (segment (start 127.635 78.74) (end 127 78.74) (width 1) (layer F.Cu) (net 3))
 (segment (start 122.935 82.55) (end 120.65 82.55) (width 1) (layer F.Cu) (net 4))
 (segment (start 120.65 82.55) (end 119.65 82.55) (width 1) (layer F.Cu) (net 4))
 (segment (start 115.57 90.17) (end 115.57 83.82) (width 1) (layer F.Cu) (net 4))
 (segment (start 116.84 82.55) (end 119.65 82.55) (width 1) (layer F.Cu) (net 4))
 (segment (start 115.57 83.82) (end 116.84 82.55) (width 1) (layer F.Cu) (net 4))
 (segment (start 122.935 93.98) (end 120.65 93.98) (width 1) (layer F.Cu) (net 5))
 (segment (start 118.044873 95.25) (end 119.314873 93.98) (width 1) (layer F.Cu) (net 5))
 (segment (start 115.57 95.25) (end 118.044873 95.25) (width 1) (layer F.Cu) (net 5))
 (segment (start 119.314873 93.98) (end 120.65 93.98) (width 1) (layer F.Cu) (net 5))
 (segment (start 122.935 105.41) (end 120.65 105.41) (width 1) (layer F.Cu) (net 6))
 (segment (start 118.11 105.41) (end 120.65 105.41) (width 1) (layer F.Cu) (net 6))
 (segment (start 115.57 100.33) (end 115.57 104.14) (width 1) (layer F.Cu) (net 6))
 (segment (start 115.57 104.14) (end 116.84 105.41) (width 1) (layer F.Cu) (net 6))
 (segment (start 116.84 105.41) (end 118.11 105.41) (width 1) (layer F.Cu) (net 6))
 (segment (start 120.65 72.39) (end 122.935 72.39) (width 1) (layer F.Cu) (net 7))
 (segment (start 115.57 76.2) (end 118.11 76.2) (width 1) (layer F.Cu) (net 7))
 (segment (start 118.11 76.2) (end 118.745 76.835) (width 1) (layer F.Cu) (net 7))
 (via (at 120.65 76.835) (size 1.2) (drill 0.5) (layers F.Cu B.Cu) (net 7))
 (segment (start 118.745 76.835) (end 120.65 76.835) (width 1) (layer F.Cu) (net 7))
 (via (at 120.65 70.485) (size 1.2) (drill 0.5) (layers F.Cu B.Cu) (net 7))
 (segment (start 120.65 76.835) (end 120.65 70.485) (width 0.6) (layer B.Cu) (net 7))
 (segment (start 120.65 70.485) (end 120.65 72.39) (width 1) (layer F.Cu) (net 7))
 (segment (start 134.89 82.87) (end 134.89 82.82) (width 1) (layer F.Cu) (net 8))
 (segment (start 134.62 82.55) (end 132.08 82.55) (width 1) (layer F.Cu) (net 8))
 (segment (start 134.89 82.82) (end 134.62 82.55) (width 1) (layer F.Cu) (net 8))
 (segment (start 129.54 85.09) (end 129.54 82.55) (width 1) (layer F.Cu) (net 8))
 (segment (start 129.54 82.55) (end 132.08 82.55) (width 1) (layer F.Cu) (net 8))
 (segment (start 129.54 82.55) (end 125.985 82.55) (width 1) (layer F.Cu) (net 8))
 (segment (start 134.89 94.3) (end 134.89 94.25) (width 1) (layer F.Cu) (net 13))
 (segment (start 134.62 93.98) (end 132.08 93.98) (width 1) (layer F.Cu) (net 13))
 (segment (start 134.89 94.25) (end 134.62 93.98) (width 1) (layer F.Cu) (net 13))
 (segment (start 129.54 93.98) (end 132.08 93.98) (width 1) (layer F.Cu) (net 13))
 (segment (start 129.54 96.52) (end 129.54 93.98) (width 1) (layer F.Cu) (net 13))
 (segment (start 125.985 93.98) (end 129.54 93.98) (width 1) (layer F.Cu) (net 13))
 (segment (start 132.4 105.73) (end 132.08 105.41) (width 0.6) (layer F.Cu) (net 14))
 (segment (start 129.54 105.41) (end 129.54 107.95) (width 1) (layer F.Cu) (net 14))
 (segment (start 129.54 105.41) (end 132.08 105.41) (width 1) (layer F.Cu) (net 14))
 (segment (start 125.985 105.41) (end 129.54 105.41) (width 1) (layer F.Cu) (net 14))
 (segment (start 134.57 105.41) (end 134.89 105.73) (width 1) (layer F.Cu) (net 14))
 (segment (start 132.08 105.41) (end 134.57 105.41) (width 1) (layer F.Cu) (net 14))
 (segment (start 142.24 104.51) (end 142.24 105.41) (width 0.6) (layer F.Cu) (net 19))
 (segment (start 129.54 91.44) (end 132.08 91.44) (width 1) (layer F.Cu) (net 19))
 (segment (start 135.89 87.63) (end 142.24 87.63) (width 1) (layer F.Cu) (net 19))
 (segment (start 132.08 91.44) (end 135.89 87.63) (width 1) (layer F.Cu) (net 19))
 (segment (start 139.7 102.87) (end 140.6 102.87) (width 1) (layer F.Cu) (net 19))
 (segment (start 129.54 102.87) (end 139.7 102.87) (width 1) (layer F.Cu) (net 19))
 (segment (start 146.05 102.87) (end 148.59 100.33) (width 1) (layer F.Cu) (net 19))
 (segment (start 142.24 105.41) (end 142.24 102.87) (width 1) (layer F.Cu) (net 19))
 (segment (start 139.7 102.87) (end 142.24 102.87) (width 1) (layer F.Cu) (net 19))
 (segment (start 142.24 102.87) (end 146.05 102.87) (width 1) (layer F.Cu) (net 19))
 (segment (start 148.59 100.33) (end 148.59 86.36) (width 1) (layer F.Cu) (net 19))
 (segment (start 147.32 85.09) (end 143.51 85.09) (width 1) (layer F.Cu) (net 19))
 (segment (start 143.51 85.09) (end 142.24 86.36) (width 1) (layer F.Cu) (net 19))
 (segment (start 142.24 86.36) (end 142.24 87.63) (width 1) (layer F.Cu) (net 19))
 (segment (start 148.59 68.58) (end 147.32 67.31) (width 1) (layer F.Cu) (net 19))
 (segment (start 142.24 69.85) (end 142.24 68.58) (width 1) (layer F.Cu) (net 19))
 (segment (start 142.24 68.58) (end 143.51 67.31) (width 1) (layer F.Cu) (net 19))
 (segment (start 143.51 67.31) (end 147.32 67.31) (width 1) (layer F.Cu) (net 19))
 (segment (start 147.32 85.09) (end 148.59 85.09) (width 1) (layer F.Cu) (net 19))
 (segment (start 148.59 86.36) (end 148.59 85.09) (width 1) (layer F.Cu) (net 19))
 (segment (start 148.59 85.09) (end 148.59 68.58) (width 1) (layer F.Cu) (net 19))
 (segment (start 129.54 80.01) (end 132.08 80.01) (width 1) (layer F.Cu) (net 19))
 (segment (start 132.08 80.01) (end 134.62 77.47) (width 1) (layer F.Cu) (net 19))
 (segment (start 125.985 72.39) (end 134.62 72.39) (width 1) (layer F.Cu) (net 19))
 (segment (start 134.62 77.47) (end 134.62 72.39) (width 1) (layer F.Cu) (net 19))
 (segment (start 134.62 72.39) (end 141.605 72.39) (width 1) (layer F.Cu) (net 19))
 (segment (start 142.24 71.755) (end 142.24 69.85) (width 1) (layer F.Cu) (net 19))
 (segment (start 141.605 72.39) (end 142.24 71.755) (width 1) (layer F.Cu) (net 19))
 (segment (start 136.89 83.82) (end 136.89 80.28) (width 1) (layer F.Cu) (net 20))
 (segment (start 138.43 78.74) (end 144.78 78.74) (width 1) (layer F.Cu) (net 20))
 (segment (start 136.89 80.28) (end 138.43 78.74) (width 1) (layer F.Cu) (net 20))
 (segment (start 144.78 76.2) (end 144.78 69.85) (width 1) (layer F.Cu) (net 21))
 (segment (start 140.97 96.52) (end 144.78 96.52) (width 1) (layer F.Cu) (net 22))
 (segment (start 136.89 95.25) (end 139.7 95.25) (width 1) (layer F.Cu) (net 22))
 (segment (start 139.7 95.25) (end 140.97 96.52) (width 1) (layer F.Cu) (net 22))
 (segment (start 144.78 87.63) (end 144.78 93.98) (width 1) (layer F.Cu) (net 23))
 (segment (start 144.78 111.76) (end 144.78 105.41) (width 1) (layer F.Cu) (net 1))
 (segment (start 136.89 106.68) (end 136.89 110.22) (width 1) (layer F.Cu) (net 2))
 (segment (start 140.97 114.3) (end 144.78 114.3) (width 1) (layer F.Cu) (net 2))
 (segment (start 136.89 110.22) (end 140.97 114.3) (width 1) (layer F.Cu) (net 2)))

